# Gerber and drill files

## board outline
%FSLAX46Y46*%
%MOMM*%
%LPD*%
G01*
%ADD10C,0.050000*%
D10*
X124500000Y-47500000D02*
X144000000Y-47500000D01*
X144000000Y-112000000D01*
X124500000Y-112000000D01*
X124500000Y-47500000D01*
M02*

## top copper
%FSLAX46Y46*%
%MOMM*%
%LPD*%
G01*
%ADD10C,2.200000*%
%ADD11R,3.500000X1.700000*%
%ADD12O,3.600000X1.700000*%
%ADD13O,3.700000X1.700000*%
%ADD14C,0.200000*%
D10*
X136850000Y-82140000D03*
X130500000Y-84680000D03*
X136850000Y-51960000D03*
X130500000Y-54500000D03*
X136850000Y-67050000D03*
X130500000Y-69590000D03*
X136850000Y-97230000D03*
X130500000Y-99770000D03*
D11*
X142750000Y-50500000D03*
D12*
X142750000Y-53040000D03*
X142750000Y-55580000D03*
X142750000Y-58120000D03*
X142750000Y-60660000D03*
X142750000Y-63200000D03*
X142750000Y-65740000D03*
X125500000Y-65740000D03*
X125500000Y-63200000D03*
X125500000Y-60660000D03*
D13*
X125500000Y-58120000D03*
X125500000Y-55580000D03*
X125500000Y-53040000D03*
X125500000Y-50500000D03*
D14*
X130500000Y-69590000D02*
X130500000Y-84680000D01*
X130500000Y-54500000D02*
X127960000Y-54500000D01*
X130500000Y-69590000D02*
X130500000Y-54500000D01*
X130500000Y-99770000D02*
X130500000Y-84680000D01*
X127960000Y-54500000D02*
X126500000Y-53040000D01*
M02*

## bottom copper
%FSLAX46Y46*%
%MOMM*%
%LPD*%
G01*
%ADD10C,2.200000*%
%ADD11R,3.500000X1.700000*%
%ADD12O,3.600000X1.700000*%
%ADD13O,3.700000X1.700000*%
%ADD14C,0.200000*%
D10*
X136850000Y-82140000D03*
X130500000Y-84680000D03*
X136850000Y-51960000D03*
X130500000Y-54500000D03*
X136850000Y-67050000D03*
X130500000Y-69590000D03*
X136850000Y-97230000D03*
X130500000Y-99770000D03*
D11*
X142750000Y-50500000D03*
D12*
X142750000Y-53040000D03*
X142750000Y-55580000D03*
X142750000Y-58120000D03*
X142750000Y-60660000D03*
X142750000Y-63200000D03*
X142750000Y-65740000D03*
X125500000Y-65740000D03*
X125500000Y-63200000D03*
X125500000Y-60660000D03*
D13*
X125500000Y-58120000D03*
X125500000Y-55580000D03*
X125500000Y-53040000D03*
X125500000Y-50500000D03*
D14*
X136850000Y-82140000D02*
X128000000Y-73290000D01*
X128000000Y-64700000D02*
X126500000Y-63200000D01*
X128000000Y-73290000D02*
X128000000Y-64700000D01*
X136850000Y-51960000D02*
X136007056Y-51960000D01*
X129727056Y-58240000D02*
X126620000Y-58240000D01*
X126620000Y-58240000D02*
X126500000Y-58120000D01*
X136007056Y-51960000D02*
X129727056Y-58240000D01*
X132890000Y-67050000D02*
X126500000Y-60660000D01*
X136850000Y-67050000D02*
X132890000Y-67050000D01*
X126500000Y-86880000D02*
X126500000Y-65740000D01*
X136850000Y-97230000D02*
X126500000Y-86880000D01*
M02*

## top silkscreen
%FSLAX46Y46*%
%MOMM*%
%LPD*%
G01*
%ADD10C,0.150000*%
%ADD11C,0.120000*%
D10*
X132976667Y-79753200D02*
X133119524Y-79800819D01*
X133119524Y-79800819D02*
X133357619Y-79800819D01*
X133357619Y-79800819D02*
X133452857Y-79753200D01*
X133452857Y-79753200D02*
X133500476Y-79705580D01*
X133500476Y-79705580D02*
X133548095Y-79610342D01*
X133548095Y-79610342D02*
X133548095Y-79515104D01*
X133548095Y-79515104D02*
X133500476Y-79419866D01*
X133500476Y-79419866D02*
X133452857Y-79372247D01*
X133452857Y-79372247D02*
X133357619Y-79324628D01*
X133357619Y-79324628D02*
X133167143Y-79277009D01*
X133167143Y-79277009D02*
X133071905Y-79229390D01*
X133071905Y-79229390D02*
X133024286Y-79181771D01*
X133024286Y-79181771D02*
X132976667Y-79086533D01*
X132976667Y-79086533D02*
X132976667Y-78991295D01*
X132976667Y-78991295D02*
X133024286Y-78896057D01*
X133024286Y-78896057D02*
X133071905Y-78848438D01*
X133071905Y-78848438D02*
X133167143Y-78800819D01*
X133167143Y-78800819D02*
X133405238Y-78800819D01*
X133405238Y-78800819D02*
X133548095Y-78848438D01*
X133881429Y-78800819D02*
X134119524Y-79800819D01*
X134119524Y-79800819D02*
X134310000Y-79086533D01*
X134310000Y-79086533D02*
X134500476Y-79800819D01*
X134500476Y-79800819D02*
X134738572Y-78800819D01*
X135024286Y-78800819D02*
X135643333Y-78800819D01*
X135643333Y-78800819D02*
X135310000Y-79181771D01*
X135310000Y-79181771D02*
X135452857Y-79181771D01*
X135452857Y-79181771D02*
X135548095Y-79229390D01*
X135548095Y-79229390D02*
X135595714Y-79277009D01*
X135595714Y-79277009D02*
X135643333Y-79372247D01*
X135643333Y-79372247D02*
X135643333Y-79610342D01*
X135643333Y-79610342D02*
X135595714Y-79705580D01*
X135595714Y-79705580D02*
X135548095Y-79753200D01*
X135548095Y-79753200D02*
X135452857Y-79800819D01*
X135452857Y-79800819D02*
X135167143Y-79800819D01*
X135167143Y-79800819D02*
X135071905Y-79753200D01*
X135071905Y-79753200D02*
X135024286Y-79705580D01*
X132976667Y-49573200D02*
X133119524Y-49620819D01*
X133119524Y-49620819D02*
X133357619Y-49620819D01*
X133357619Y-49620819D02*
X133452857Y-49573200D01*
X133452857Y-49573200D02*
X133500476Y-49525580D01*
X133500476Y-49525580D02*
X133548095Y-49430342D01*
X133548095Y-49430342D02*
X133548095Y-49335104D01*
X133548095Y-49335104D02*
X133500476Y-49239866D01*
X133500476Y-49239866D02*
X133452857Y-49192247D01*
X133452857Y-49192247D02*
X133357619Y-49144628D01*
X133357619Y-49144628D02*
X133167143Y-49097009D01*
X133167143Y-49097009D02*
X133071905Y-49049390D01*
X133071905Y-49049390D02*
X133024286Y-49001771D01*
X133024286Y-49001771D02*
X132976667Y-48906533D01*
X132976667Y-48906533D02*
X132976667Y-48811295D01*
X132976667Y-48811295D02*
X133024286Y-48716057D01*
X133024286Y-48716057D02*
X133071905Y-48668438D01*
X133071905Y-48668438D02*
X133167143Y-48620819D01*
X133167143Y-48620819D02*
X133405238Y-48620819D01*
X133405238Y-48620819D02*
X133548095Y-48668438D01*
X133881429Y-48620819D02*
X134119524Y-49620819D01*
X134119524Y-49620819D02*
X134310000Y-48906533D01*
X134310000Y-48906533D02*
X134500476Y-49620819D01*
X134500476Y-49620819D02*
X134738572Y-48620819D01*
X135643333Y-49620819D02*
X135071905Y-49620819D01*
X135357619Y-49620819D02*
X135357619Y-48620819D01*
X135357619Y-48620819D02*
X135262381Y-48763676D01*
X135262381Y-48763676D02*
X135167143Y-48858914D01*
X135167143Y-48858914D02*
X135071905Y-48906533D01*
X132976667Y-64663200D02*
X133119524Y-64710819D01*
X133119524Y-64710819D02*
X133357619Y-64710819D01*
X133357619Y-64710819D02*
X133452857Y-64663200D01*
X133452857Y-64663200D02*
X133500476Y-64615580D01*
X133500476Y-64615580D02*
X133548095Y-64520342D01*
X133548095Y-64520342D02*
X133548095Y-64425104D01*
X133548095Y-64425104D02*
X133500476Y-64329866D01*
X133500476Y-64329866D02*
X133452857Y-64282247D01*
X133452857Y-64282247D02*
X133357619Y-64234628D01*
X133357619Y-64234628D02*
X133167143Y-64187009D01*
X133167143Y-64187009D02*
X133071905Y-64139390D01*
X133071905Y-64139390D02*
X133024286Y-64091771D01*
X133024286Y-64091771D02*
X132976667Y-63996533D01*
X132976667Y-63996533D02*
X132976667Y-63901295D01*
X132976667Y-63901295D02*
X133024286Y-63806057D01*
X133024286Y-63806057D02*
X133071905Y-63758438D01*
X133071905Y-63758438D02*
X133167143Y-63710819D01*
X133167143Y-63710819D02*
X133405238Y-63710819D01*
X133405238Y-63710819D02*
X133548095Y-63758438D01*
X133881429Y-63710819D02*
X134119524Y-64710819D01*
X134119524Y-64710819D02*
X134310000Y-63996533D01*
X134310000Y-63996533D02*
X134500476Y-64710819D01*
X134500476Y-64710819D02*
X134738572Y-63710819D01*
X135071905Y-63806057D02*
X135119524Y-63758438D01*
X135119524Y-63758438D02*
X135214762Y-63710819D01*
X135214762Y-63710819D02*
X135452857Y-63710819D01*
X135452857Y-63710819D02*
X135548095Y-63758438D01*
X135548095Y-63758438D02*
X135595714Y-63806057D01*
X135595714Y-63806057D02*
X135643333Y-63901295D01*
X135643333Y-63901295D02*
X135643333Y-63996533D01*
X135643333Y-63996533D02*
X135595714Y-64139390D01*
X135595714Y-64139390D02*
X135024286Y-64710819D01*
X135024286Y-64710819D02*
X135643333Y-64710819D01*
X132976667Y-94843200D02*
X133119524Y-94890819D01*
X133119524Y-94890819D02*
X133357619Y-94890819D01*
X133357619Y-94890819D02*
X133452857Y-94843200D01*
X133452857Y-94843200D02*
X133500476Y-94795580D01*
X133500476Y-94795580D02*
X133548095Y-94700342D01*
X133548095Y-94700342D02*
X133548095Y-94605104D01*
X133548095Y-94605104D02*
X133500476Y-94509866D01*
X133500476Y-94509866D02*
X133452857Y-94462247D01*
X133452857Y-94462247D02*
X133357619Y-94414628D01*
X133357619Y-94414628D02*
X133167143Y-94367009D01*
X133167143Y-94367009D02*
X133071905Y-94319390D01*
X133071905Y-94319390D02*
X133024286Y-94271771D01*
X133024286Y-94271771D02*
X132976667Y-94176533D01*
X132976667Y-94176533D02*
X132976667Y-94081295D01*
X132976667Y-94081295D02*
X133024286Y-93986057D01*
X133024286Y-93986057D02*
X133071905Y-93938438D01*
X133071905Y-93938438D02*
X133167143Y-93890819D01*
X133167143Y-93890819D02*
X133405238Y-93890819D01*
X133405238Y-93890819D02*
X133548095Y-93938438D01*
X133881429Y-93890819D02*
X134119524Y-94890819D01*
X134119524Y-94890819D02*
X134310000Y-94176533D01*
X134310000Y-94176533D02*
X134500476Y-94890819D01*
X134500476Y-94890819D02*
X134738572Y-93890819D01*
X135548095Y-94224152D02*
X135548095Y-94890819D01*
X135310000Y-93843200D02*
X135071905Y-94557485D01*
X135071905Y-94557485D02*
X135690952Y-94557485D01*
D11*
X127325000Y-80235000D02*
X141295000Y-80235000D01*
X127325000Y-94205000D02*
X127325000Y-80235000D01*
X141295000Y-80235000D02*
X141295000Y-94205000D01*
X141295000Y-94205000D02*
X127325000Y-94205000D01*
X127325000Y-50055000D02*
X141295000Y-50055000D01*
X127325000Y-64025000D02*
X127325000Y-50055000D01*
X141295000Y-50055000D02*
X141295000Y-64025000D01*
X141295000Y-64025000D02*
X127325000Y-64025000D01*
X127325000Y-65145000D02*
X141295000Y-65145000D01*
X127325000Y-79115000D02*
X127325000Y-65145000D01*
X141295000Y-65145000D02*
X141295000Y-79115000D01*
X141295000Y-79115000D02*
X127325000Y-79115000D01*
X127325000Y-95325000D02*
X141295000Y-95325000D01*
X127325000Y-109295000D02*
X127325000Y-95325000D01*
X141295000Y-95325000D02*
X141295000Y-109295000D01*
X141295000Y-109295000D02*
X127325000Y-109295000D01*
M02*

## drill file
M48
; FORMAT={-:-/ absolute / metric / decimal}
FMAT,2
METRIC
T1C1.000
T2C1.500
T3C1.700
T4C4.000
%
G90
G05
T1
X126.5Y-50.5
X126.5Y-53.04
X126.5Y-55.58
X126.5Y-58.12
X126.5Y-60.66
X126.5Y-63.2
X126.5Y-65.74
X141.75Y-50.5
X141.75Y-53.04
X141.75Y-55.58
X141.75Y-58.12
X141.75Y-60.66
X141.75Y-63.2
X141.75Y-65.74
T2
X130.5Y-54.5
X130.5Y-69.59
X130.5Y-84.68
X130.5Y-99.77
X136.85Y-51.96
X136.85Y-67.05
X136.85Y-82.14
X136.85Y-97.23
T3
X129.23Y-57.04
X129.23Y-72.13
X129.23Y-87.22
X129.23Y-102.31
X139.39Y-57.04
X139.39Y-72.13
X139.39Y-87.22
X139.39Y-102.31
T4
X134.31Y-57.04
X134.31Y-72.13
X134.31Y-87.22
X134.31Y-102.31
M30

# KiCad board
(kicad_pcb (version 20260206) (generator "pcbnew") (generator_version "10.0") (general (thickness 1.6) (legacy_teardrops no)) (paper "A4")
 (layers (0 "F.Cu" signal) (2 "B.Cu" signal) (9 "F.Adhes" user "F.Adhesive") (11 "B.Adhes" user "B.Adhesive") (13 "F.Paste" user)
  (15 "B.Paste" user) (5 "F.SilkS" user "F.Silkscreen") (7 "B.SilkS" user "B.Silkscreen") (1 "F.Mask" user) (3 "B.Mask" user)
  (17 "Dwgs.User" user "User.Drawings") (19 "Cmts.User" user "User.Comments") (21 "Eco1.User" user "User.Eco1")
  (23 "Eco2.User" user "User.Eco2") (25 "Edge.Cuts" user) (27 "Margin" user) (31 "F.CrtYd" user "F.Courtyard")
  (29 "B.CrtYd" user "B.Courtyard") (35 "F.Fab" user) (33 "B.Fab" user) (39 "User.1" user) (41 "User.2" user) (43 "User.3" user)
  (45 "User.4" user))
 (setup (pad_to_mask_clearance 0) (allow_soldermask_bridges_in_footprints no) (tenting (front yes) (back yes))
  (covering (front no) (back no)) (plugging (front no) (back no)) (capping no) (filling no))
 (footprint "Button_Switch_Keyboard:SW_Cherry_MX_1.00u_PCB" (layer "F.Cu") (at 136.85 82.14)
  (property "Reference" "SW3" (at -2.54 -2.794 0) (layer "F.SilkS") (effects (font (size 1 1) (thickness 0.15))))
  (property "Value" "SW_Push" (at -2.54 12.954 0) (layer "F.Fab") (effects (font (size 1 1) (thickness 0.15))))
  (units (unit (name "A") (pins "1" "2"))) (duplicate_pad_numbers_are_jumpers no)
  (fp_line (start -9.525 -1.905) (end 4.445 -1.905) (stroke (width 0.12) (type solid)) (layer "F.SilkS"))
  (fp_line (start -9.525 12.065) (end -9.525 -1.905) (stroke (width 0.12) (type solid)) (layer "F.SilkS"))
  (fp_line (start 4.445 -1.905) (end 4.445 12.065) (stroke (width 0.12) (type solid)) (layer "F.SilkS"))
  (fp_line (start 4.445 12.065) (end -9.525 12.065) (stroke (width 0.12) (type solid)) (layer "F.SilkS"))
  (pad "" np_thru_hole circle (at -7.62 5.08) (size 1.7 1.7) (drill 1.7) (layers "*.Cu" "*.Mask"))
  (pad "" np_thru_hole circle (at -2.54 5.08) (size 4 4) (drill 4) (layers "*.Cu" "*.Mask"))
  (pad "" np_thru_hole circle (at 2.54 5.08) (size 1.7 1.7) (drill 1.7) (layers "*.Cu" "*.Mask"))
  (pad "1" thru_hole circle (at 0 0) (size 2.2 2.2) (drill 1.5) (layers "*.Cu" "*.Mask") (remove_unused_layers no)
   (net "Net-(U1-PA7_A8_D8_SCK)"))
  (pad "2" thru_hole circle (at -6.35 2.54) (size 2.2 2.2) (drill 1.5) (layers "*.Cu" "*.Mask") (remove_unused_layers no) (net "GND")))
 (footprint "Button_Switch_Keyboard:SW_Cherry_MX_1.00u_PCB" (layer "F.Cu") (at 136.85 51.96)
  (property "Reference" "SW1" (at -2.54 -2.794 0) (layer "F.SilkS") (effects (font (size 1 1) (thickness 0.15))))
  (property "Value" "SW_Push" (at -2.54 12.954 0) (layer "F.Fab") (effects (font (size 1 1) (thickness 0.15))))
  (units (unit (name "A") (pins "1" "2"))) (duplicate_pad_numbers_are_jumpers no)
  (fp_line (start -9.525 -1.905) (end 4.445 -1.905) (stroke (width 0.12) (type solid)) (layer "F.SilkS"))
  (fp_line (start -9.525 12.065) (end -9.525 -1.905) (stroke (width 0.12) (type solid)) (layer "F.SilkS"))
  (fp_line (start 4.445 -1.905) (end 4.445 12.065) (stroke (width 0.12) (type solid)) (layer "F.SilkS"))
  (fp_line (start 4.445 12.065) (end -9.525 12.065) (stroke (width 0.12) (type solid)) (layer "F.SilkS"))
  (pad "" np_thru_hole circle (at -7.62 5.08) (size 1.7 1.7) (drill 1.7) (layers "*.Cu" "*.Mask"))
  (pad "" np_thru_hole circle (at -2.54 5.08) (size 4 4) (drill 4) (layers "*.Cu" "*.Mask"))
  (pad "" np_thru_hole circle (at 2.54 5.08) (size 1.7 1.7) (drill 1.7) (layers "*.Cu" "*.Mask"))
  (pad "1" thru_hole circle (at 0 0) (size 2.2 2.2) (drill 1.5) (layers "*.Cu" "*.Mask") (remove_unused_layers no)
   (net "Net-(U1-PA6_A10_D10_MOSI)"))
  (pad "2" thru_hole circle (at -6.35 2.54) (size 2.2 2.2) (drill 1.5) (layers "*.Cu" "*.Mask") (remove_unused_layers no) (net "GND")))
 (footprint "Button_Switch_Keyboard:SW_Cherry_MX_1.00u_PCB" (layer "F.Cu") (at 136.85 67.05)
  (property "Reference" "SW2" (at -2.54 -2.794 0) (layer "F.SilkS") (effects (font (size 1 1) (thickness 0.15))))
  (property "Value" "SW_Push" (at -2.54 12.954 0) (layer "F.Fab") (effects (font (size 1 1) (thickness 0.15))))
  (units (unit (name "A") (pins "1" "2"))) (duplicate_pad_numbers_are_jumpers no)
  (fp_line (start -9.525 -1.905) (end 4.445 -1.905) (stroke (width 0.12) (type solid)) (layer "F.SilkS"))
  (fp_line (start -9.525 12.065) (end -9.525 -1.905) (stroke (width 0.12) (type solid)) (layer "F.SilkS"))
  (fp_line (start 4.445 -1.905) (end 4.445 12.065) (stroke (width 0.12) (type solid)) (layer "F.SilkS"))
  (fp_line (start 4.445 12.065) (end -9.525 12.065) (stroke (width 0.12) (type solid)) (layer "F.SilkS"))
  (pad "" np_thru_hole circle (at -7.62 5.08) (size 1.7 1.7) (drill 1.7) (layers "*.Cu" "*.Mask"))
  (pad "" np_thru_hole circle (at -2.54 5.08) (size 4 4) (drill 4) (layers "*.Cu" "*.Mask"))
  (pad "" np_thru_hole circle (at 2.54 5.08) (size 1.7 1.7) (drill 1.7) (layers "*.Cu" "*.Mask"))
  (pad "1" thru_hole circle (at 0 0) (size 2.2 2.2) (drill 1.5) (layers "*.Cu" "*.Mask") (remove_unused_layers no)
   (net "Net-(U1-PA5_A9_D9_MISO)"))
  (pad "2" thru_hole circle (at -6.35 2.54) (size 2.2 2.2) (drill 1.5) (layers "*.Cu" "*.Mask") (remove_unused_layers no) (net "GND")))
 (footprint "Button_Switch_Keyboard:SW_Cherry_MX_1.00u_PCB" (layer "F.Cu") (at 136.85 97.23)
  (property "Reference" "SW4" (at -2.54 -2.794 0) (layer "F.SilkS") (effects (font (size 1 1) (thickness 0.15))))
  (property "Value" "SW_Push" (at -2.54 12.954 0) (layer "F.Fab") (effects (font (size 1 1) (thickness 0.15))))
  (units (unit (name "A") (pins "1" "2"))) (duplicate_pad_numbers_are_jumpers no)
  (fp_line (start -9.525 -1.905) (end 4.445 -1.905) (stroke (width 0.12) (type solid)) (layer "F.SilkS"))
  (fp_line (start -9.525 12.065) (end -9.525 -1.905) (stroke (width 0.12) (type solid)) (layer "F.SilkS"))
  (fp_line (start 4.445 -1.905) (end 4.445 12.065) (stroke (width 0.12) (type solid)) (layer "F.SilkS"))
  (fp_line (start 4.445 12.065) (end -9.525 12.065) (stroke (width 0.12) (type solid)) (layer "F.SilkS"))
  (pad "" np_thru_hole circle (at -7.62 5.08) (size 1.7 1.7) (drill 1.7) (layers "*.Cu" "*.Mask"))
  (pad "" np_thru_hole circle (at -2.54 5.08) (size 4 4) (drill 4) (layers "*.Cu" "*.Mask"))
  (pad "" np_thru_hole circle (at 2.54 5.08) (size 1.7 1.7) (drill 1.7) (layers "*.Cu" "*.Mask"))
  (pad "1" thru_hole circle (at 0 0) (size 2.2 2.2) (drill 1.5) (layers "*.Cu" "*.Mask") (remove_unused_layers no)
   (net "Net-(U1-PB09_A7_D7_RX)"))
  (pad "2" thru_hole circle (at -6.35 2.54) (size 2.2 2.2) (drill 1.5) (layers "*.Cu" "*.Mask") (remove_unused_layers no) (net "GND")))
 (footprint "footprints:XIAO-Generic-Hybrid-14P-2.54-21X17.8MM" (layer "B.Cu") (at 134.125 58.12 180)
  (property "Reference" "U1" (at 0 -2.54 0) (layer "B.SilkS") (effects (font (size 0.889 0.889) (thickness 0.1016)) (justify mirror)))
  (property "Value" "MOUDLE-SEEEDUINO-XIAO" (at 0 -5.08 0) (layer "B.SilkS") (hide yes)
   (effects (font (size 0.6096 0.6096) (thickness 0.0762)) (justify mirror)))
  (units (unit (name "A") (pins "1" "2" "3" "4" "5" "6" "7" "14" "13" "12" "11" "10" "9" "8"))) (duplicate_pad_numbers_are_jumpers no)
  (pad "1" thru_hole rect (at -7.625 7.62 180) (size 3.5 1.7) (drill 1 (offset -1 0)) (layers "*.Cu" "*.Mask") (remove_unused_layers no)
   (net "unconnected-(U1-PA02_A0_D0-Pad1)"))
  (pad "2" thru_hole oval (at -7.625 5.08 180) (size 3.6 1.7) (drill 1 (offset -1 0)) (layers "*.Cu" "*.Mask") (remove_unused_layers no)
   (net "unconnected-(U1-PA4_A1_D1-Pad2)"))
  (pad "3" thru_hole oval (at -7.625 2.54 180) (size 3.6 1.7) (drill 1 (offset -1 0)) (layers "*.Cu" "*.Mask") (remove_unused_layers no)
   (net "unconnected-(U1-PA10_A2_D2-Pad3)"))
  (pad "4" thru_hole oval (at -7.625 0 180) (size 3.6 1.7) (drill 1 (offset -1 0)) (layers "*.Cu" "*.Mask") (remove_unused_layers no)
   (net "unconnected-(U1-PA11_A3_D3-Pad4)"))
  (pad "5" thru_hole oval (at -7.625 -2.54 180) (size 3.6 1.7) (drill 1 (offset -1 0)) (layers "*.Cu" "*.Mask") (remove_unused_layers no)
   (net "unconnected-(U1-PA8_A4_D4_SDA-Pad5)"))
  (pad "6" thru_hole oval (at -7.625 -5.08) (size 3.6 1.7) (drill 1 (offset 1 0)) (layers "*.Cu" "*.Mask") (remove_unused_layers no)
   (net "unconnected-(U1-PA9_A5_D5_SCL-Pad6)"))
  (pad "7" thru_hole oval (at -7.625 -7.62 180) (size 3.6 1.7) (drill 1 (offset -1 0)) (layers "*.Cu" "*.Mask") (remove_unused_layers no)
   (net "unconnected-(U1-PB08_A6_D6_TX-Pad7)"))
  (pad "8" thru_hole oval (at 7.625 -7.62 180) (size 3.6 1.7) (drill 1 (offset 1 0)) (layers "*.Cu" "*.Mask") (remove_unused_layers no)
   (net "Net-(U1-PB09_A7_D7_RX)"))
  (pad "9" thru_hole oval (at 7.625 -5.08 180) (size 3.6 1.7) (drill 1 (offset 1 0)) (layers "*.Cu" "*.Mask") (remove_unused_layers no)
   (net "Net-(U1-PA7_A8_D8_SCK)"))
  (pad "10" thru_hole oval (at 7.625 -2.54 180) (size 3.6 1.7) (drill 1 (offset 1 0)) (layers "*.Cu" "*.Mask") (remove_unused_layers no)
   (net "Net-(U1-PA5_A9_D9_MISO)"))
  (pad "11" thru_hole oval (at 7.625 0 180) (size 3.7 1.7) (drill 1 (offset 1 0)) (layers "*.Cu" "*.Mask") (remove_unused_layers no)
   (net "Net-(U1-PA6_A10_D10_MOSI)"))
  (pad "12" thru_hole oval (at 7.625 2.54 180) (size 3.7 1.7) (drill 1 (offset 1 0)) (layers "*.Cu" "*.Mask") (remove_unused_layers no)
   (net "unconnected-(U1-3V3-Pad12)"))
  (pad "13" thru_hole oval (at 7.625 5.08 180) (size 3.7 1.7) (drill 1 (offset 1 0)) (layers "*.Cu" "*.Mask") (remove_unused_layers no)
   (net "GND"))
  (pad "14" thru_hole oval (at 7.625 7.62 180) (size 3.7 1.7) (drill 1 (offset 1 0)) (layers "*.Cu" "*.Mask") (remove_unused_layers no)
   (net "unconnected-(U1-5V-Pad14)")))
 (gr_rect (start 124.5 47.5) (end 144 112) (stroke (width 0.05) (type default)) (fill no) (layer "Edge.Cuts"))
 (segment (start 136.85 82.14) (end 128 73.29) (width 0.2) (layer "B.Cu") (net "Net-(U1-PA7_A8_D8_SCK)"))
 (segment (start 128 64.7) (end 126.5 63.2) (width 0.2) (layer "B.Cu") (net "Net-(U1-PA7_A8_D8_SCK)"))
 (segment (start 128 73.29) (end 128 64.7) (width 0.2) (layer "B.Cu") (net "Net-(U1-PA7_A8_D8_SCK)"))
 (segment (start 130.5 69.59) (end 130.5 84.68) (width 0.2) (layer "F.Cu") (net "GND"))
 (segment (start 130.5 54.5) (end 127.96 54.5) (width 0.2) (layer "F.Cu") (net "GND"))
 (segment (start 130.5 69.59) (end 130.5 54.5) (width 0.2) (layer "F.Cu") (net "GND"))
 (segment (start 130.5 99.77) (end 130.5 84.68) (width 0.2) (layer "F.Cu") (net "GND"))
 (segment (start 127.96 54.5) (end 126.5 53.04) (width 0.2) (layer "F.Cu") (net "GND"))
 (segment (start 136.85 51.96) (end 136.007056 51.96) (width 0.2) (layer "B.Cu") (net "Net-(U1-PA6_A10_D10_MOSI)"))
 (segment (start 129.727056 58.24) (end 126.62 58.24) (width 0.2) (layer "B.Cu") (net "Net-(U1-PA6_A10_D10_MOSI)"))
 (segment (start 126.62 58.24) (end 126.5 58.12) (width 0.2) (layer "B.Cu") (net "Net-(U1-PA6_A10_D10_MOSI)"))
 (segment (start 136.007056 51.96) (end 129.727056 58.24) (width 0.2) (layer "B.Cu") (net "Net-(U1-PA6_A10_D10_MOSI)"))
 (segment (start 132.89 67.05) (end 126.5 60.66) (width 0.2) (layer "B.Cu") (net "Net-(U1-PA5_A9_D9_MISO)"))
 (segment (start 136.85 67.05) (end 132.89 67.05) (width 0.2) (layer "B.Cu") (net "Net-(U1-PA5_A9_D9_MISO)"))
 (segment (start 126.5 86.88) (end 126.5 65.74) (width 0.2) (layer "B.Cu") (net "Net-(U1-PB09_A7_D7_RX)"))
 (segment (start 136.85 97.23) (end 126.5 86.88) (width 0.2) (layer "B.Cu") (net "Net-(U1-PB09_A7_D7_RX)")))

